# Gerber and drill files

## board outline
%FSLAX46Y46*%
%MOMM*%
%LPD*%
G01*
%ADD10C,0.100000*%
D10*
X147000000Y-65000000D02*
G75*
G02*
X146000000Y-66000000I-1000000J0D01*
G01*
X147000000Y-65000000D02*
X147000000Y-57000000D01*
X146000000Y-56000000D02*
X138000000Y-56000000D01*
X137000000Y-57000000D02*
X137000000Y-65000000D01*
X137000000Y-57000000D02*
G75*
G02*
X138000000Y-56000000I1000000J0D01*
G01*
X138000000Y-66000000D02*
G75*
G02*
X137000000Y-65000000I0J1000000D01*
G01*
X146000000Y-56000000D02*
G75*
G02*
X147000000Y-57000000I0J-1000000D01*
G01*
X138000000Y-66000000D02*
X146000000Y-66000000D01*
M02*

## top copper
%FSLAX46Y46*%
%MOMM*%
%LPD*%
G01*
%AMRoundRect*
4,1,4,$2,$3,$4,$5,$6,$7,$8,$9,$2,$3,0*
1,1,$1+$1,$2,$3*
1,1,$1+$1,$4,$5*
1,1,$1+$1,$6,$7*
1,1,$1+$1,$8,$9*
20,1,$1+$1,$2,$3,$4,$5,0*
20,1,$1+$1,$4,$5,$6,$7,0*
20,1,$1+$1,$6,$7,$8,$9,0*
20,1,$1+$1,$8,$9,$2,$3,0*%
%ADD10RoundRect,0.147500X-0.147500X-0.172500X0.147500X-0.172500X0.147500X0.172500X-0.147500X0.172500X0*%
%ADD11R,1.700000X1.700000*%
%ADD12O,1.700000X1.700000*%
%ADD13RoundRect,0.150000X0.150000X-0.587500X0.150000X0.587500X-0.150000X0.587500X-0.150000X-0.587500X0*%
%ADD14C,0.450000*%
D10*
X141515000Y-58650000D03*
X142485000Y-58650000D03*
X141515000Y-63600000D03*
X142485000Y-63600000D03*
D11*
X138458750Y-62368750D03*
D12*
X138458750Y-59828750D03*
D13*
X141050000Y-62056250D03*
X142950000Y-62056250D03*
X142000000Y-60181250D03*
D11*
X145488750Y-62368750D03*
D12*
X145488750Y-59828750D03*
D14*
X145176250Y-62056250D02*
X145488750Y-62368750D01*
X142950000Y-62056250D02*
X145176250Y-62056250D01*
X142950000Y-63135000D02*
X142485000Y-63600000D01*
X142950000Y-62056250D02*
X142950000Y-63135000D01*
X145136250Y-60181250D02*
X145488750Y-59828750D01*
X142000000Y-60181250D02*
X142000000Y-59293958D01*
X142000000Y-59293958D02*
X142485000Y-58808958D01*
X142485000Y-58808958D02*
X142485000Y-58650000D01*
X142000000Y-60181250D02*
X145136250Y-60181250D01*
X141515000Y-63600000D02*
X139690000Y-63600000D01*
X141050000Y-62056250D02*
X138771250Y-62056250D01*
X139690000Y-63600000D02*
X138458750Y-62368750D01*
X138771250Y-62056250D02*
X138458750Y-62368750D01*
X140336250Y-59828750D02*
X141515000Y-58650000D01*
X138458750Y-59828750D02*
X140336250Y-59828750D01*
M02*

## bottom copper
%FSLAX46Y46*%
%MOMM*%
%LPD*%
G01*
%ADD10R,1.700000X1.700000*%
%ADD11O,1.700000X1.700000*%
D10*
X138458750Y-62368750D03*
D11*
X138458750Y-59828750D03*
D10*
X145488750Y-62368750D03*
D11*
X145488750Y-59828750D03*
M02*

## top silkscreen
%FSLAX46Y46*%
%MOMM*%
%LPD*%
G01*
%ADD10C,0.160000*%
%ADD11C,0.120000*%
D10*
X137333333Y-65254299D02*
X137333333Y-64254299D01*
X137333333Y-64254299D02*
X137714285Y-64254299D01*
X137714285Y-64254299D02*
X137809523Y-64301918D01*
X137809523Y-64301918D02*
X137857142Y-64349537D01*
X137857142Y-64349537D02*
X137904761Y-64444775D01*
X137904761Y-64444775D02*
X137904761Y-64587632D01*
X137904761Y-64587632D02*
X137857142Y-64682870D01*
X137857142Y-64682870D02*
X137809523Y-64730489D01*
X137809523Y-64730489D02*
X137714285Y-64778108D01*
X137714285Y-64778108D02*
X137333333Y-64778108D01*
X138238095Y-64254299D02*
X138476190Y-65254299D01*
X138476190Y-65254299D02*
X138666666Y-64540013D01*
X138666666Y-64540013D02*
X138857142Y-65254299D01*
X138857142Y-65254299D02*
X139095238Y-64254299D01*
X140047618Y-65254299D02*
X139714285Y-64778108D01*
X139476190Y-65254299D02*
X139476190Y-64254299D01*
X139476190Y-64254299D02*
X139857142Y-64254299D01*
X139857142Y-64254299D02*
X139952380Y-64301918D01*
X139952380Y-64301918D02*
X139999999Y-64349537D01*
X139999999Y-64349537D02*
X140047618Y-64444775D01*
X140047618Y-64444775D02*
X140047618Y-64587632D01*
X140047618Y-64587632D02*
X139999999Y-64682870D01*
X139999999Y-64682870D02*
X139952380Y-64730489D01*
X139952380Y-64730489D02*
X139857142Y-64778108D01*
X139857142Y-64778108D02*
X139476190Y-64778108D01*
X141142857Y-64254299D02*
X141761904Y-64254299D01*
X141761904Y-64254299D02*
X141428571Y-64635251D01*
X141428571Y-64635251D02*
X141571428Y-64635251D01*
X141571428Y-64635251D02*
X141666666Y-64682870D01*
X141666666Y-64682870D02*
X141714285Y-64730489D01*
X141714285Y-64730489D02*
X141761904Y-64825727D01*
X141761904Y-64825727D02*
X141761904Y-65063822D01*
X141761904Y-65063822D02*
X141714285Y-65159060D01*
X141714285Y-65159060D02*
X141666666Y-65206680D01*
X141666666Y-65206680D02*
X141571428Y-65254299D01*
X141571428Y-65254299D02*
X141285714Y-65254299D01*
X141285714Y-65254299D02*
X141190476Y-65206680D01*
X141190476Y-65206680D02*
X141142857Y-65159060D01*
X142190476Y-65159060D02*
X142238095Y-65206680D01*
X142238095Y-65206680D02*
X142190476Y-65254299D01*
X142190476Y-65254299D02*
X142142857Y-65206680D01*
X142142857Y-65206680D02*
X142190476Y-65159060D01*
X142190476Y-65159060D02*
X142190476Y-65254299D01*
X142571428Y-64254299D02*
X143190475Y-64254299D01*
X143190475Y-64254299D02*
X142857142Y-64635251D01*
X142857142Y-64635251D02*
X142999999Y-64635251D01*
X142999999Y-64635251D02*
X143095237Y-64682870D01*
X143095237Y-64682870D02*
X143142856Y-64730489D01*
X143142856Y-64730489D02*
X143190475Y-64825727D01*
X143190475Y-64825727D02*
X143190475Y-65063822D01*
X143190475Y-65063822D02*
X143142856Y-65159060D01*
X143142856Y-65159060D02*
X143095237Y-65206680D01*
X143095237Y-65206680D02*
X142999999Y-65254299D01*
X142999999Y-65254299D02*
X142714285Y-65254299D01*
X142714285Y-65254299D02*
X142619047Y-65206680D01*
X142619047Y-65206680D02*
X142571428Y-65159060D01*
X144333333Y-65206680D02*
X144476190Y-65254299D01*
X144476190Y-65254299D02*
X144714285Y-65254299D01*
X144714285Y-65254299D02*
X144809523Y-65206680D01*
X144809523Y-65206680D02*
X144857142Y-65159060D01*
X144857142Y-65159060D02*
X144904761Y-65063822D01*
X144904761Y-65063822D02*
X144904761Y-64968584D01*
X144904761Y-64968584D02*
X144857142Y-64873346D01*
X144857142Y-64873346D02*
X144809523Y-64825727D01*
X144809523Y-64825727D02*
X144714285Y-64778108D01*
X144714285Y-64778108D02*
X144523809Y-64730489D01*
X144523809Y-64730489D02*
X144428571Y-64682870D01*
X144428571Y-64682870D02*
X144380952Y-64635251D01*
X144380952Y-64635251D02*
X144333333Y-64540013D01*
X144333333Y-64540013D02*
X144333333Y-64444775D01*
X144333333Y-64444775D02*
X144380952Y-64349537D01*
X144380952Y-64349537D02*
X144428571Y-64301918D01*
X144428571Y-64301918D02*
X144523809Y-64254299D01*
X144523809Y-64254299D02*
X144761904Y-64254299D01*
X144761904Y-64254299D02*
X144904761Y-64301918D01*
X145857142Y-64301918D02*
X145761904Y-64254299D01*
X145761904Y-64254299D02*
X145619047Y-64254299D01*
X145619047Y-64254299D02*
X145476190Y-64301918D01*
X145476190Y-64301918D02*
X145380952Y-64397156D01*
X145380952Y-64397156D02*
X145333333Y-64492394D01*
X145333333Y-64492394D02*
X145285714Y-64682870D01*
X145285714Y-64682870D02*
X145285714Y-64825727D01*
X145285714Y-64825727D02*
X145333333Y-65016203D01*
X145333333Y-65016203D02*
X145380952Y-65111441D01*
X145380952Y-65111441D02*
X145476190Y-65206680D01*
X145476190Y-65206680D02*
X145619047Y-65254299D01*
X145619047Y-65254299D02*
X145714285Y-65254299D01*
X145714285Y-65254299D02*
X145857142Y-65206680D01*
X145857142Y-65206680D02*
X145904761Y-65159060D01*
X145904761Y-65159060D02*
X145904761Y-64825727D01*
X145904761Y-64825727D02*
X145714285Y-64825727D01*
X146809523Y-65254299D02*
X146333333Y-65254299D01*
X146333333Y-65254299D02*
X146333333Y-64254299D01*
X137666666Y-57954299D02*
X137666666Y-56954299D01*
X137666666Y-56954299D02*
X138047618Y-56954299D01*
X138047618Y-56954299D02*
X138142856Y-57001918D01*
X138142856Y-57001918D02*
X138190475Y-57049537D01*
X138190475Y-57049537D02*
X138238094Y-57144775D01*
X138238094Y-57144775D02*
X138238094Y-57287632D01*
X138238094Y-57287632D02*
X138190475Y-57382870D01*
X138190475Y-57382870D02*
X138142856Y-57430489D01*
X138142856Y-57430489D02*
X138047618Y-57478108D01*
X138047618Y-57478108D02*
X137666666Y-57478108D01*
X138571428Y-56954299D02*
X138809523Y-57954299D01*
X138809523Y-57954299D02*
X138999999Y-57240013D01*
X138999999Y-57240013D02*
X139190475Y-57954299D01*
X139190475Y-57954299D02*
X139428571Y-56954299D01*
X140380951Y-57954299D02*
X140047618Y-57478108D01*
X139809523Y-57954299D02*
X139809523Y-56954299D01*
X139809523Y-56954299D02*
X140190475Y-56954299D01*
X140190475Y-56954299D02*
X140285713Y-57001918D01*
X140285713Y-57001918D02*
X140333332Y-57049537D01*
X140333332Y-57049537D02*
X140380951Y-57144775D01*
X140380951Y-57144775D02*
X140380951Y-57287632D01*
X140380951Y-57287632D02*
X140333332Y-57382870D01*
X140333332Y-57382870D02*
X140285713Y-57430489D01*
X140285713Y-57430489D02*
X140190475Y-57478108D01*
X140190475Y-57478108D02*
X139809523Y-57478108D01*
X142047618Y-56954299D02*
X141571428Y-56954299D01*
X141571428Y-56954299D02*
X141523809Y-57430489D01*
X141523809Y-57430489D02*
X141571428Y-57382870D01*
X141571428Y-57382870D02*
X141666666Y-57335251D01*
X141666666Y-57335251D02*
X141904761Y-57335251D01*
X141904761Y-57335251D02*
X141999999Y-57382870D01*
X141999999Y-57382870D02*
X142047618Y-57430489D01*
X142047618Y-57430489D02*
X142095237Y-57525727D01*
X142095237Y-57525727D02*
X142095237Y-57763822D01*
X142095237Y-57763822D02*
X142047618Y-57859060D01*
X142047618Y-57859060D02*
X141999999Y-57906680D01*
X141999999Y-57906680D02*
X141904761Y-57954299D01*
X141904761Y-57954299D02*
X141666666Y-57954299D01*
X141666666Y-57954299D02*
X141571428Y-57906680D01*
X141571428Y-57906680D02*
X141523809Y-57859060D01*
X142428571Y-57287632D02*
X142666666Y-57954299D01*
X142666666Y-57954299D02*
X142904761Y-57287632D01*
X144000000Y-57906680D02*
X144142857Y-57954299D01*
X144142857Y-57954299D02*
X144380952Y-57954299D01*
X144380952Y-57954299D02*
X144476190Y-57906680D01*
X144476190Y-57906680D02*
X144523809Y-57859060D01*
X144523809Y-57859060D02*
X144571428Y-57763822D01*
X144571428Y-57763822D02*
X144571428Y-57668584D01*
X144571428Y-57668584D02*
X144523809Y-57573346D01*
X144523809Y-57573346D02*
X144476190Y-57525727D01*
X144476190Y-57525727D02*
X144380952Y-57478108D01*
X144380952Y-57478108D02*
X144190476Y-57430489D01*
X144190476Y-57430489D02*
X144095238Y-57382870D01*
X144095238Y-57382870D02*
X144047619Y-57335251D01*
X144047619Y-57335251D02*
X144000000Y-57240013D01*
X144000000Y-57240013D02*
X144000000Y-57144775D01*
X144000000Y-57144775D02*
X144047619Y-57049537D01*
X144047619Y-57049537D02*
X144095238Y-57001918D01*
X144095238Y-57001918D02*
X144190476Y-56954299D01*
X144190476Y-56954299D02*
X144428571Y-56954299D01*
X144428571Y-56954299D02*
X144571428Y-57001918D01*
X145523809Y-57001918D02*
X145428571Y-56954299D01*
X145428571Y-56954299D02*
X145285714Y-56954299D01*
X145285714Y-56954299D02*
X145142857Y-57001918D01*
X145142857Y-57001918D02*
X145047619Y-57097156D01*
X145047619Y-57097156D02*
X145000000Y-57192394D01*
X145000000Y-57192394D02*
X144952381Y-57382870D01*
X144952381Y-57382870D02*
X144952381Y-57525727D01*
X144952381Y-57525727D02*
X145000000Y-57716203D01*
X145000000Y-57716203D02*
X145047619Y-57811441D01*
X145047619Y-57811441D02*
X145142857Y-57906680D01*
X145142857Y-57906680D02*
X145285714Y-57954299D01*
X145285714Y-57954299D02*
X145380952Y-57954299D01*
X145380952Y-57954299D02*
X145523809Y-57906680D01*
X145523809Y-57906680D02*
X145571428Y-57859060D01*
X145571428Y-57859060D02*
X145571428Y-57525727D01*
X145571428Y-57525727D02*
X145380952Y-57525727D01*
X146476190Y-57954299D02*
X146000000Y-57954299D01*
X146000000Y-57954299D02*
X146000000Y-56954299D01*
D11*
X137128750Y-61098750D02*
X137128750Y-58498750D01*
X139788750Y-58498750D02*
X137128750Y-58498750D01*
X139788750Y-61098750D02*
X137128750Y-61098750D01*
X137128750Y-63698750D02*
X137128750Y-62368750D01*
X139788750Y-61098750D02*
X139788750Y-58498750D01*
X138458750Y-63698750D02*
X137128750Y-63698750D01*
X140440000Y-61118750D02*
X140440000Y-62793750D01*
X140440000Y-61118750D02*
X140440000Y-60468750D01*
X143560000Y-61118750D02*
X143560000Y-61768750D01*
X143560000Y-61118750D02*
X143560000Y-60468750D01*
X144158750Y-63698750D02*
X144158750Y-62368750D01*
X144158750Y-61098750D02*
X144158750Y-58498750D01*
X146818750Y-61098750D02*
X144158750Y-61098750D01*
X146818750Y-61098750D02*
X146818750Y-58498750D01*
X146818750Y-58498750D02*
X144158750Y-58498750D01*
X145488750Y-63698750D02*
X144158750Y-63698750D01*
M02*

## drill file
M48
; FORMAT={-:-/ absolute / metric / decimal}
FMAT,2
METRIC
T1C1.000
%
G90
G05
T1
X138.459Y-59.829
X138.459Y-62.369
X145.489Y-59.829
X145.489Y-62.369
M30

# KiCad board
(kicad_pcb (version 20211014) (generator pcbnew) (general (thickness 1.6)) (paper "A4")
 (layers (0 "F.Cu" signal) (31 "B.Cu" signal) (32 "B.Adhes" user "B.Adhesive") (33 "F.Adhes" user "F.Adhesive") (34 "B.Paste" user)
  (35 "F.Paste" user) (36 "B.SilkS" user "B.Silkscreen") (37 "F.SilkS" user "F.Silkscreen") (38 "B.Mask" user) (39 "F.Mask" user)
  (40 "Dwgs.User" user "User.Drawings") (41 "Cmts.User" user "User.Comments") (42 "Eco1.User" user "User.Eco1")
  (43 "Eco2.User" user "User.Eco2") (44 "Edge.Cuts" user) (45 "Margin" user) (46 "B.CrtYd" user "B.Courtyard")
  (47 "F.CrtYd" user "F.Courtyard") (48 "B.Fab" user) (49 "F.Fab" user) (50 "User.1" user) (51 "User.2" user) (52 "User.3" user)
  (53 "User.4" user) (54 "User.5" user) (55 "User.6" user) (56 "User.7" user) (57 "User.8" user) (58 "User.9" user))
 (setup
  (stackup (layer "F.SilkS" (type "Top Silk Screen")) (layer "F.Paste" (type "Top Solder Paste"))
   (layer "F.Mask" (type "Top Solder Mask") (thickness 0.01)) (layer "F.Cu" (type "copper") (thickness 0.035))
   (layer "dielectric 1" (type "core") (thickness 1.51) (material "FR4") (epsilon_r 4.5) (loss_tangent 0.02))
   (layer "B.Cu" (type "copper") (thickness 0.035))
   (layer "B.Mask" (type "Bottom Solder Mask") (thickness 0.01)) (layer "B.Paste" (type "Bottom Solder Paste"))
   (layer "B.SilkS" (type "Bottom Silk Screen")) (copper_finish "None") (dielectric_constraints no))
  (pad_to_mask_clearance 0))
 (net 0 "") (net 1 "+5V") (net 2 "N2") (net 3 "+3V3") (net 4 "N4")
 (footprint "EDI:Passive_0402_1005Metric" (layer "F.Cu") (at 142 58.65)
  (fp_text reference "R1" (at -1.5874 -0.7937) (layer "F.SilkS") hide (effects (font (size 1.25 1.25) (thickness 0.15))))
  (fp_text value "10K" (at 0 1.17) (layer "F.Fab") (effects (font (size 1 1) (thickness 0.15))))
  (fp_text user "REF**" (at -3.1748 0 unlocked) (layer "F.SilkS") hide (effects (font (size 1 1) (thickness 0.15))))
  (pad "1" smd roundrect (at -0.485 0) (size 0.59 0.64) (layers "F.Cu" "F.Paste" "F.Mask") (roundrect_rratio 0.25) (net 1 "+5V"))
  (pad "2" smd roundrect (at 0.485 0) (size 0.59 0.64) (layers "F.Cu" "F.Paste" "F.Mask") (roundrect_rratio 0.25) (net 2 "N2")))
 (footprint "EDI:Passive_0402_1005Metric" (layer "F.Cu") (at 142 63.6)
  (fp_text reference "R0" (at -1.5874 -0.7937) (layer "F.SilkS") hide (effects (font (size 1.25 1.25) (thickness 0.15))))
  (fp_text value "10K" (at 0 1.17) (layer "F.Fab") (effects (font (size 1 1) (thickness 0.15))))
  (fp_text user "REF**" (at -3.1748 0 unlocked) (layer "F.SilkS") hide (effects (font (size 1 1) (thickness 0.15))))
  (pad "1" smd roundrect (at -0.485 0) (size 0.59 0.64) (layers "F.Cu" "F.Paste" "F.Mask") (roundrect_rratio 0.25) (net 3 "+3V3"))
  (pad "2" smd roundrect (at 0.485 0) (size 0.59 0.64) (layers "F.Cu" "F.Paste" "F.Mask") (roundrect_rratio 0.25) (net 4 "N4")))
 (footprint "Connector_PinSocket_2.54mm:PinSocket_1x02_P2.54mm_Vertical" (layer "F.Cu") (at 138.45875 62.36875 180)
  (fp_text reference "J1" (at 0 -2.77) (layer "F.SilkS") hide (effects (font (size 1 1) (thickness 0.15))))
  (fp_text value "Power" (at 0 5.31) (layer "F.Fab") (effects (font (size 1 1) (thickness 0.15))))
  (fp_line (start 1.33 1.27) (end 1.33 3.87) (layer "F.SilkS") (width 0.12))
  (fp_line (start -1.33 3.87) (end 1.33 3.87) (layer "F.SilkS") (width 0.12))
  (fp_line (start -1.33 1.27) (end 1.33 1.27) (layer "F.SilkS") (width 0.12))
  (fp_line (start 1.33 -1.33) (end 1.33 0) (layer "F.SilkS") (width 0.12))
  (fp_line (start -1.33 1.27) (end -1.33 3.87) (layer "F.SilkS") (width 0.12))
  (fp_line (start 0 -1.33) (end 1.33 -1.33) (layer "F.SilkS") (width 0.12))
  (pad "1" thru_hole rect locked (at 0 0 180) (size 1.7 1.7) (drill 1) (layers *.Cu *.Mask) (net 3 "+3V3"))
  (pad "2" thru_hole oval locked (at 0 2.54 180) (size 1.7 1.7) (drill 1) (layers *.Cu *.Mask) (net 1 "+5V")))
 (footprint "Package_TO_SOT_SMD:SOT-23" (layer "F.Cu") (at 142 61.11875 90)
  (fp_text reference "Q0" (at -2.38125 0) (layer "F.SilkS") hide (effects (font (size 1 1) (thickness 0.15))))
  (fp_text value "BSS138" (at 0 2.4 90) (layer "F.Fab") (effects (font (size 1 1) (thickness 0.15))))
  (fp_line (start 0 -1.56) (end -1.675 -1.56) (layer "F.SilkS") (width 0.12))
  (fp_line (start 0 -1.56) (end 0.65 -1.56) (layer "F.SilkS") (width 0.12))
  (fp_line (start 0 1.56) (end -0.65 1.56) (layer "F.SilkS") (width 0.12))
  (fp_line (start 0 1.56) (end 0.65 1.56) (layer "F.SilkS") (width 0.12))
  (pad "1" smd roundrect locked (at -0.9375 -0.95 90) (size 1.475 0.6) (layers "F.Cu" "F.Paste" "F.Mask") (roundrect_rratio 0.25)
   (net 3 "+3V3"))
  (pad "2" smd roundrect locked (at -0.9375 0.95 90) (size 1.475 0.6) (layers "F.Cu" "F.Paste" "F.Mask") (roundrect_rratio 0.25)
   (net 4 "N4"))
  (pad "3" smd roundrect locked (at 0.9375 0 90) (size 1.475 0.6) (layers "F.Cu" "F.Paste" "F.Mask") (roundrect_rratio 0.25) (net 2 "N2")))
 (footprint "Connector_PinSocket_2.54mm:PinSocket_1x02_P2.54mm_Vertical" (layer "F.Cu") (at 145.48875 62.36875 180)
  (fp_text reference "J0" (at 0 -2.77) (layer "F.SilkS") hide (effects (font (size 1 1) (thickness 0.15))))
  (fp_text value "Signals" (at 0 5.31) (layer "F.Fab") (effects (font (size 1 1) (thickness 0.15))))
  (fp_line (start 1.33 -1.33) (end 1.33 0) (layer "F.SilkS") (width 0.12))
  (fp_line (start 1.33 1.27) (end 1.33 3.87) (layer "F.SilkS") (width 0.12))
  (fp_line (start -1.33 1.27) (end 1.33 1.27) (layer "F.SilkS") (width 0.12))
  (fp_line (start -1.33 1.27) (end -1.33 3.87) (layer "F.SilkS") (width 0.12))
  (fp_line (start -1.33 3.87) (end 1.33 3.87) (layer "F.SilkS") (width 0.12))
  (fp_line (start 0 -1.33) (end 1.33 -1.33) (layer "F.SilkS") (width 0.12))
  (pad "1" thru_hole rect locked (at 0 0 180) (size 1.7 1.7) (drill 1) (layers *.Cu *.Mask) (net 4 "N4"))
  (pad "2" thru_hole oval locked (at 0 2.54 180) (size 1.7 1.7) (drill 1) (layers *.Cu *.Mask) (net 2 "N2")))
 (gr_arc (start 147 65) (mid 146.707107 65.707107) (end 146 66) (layer "Edge.Cuts") (width 0.1))
 (gr_line (start 147 65) (end 147 57) (layer "Edge.Cuts") (width 0.1))
 (gr_line (start 146 56) (end 138 56) (layer "Edge.Cuts") (width 0.1))
 (gr_line (start 137 57) (end 137 65) (layer "Edge.Cuts") (width 0.1))
 (gr_arc (start 137 57) (mid 137.292893 56.292893) (end 138 56) (layer "Edge.Cuts") (width 0.1))
 (gr_arc (start 138 66) (mid 137.292893 65.707107) (end 137 65) (layer "Edge.Cuts") (width 0.1))
 (gr_arc (start 146 56) (mid 146.707107 56.292893) (end 147 57) (layer "Edge.Cuts") (width 0.1))
 (gr_line (start 138 66) (end 146 66) (layer "Edge.Cuts") (width 0.1))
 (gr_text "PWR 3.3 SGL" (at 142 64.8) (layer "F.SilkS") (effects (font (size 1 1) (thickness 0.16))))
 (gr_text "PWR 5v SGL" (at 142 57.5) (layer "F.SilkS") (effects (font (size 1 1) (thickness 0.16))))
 (segment (start 145.17625 62.05625) (end 145.48875 62.36875) (width 0.45) (layer "F.Cu") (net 4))
 (segment (start 142.95 62.05625) (end 145.17625 62.05625) (width 0.45) (layer "F.Cu") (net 4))
 (segment (start 142.95 63.135) (end 142.485 63.6) (width 0.45) (layer "F.Cu") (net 4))
 (segment (start 142.95 62.05625) (end 142.95 63.135) (width 0.45) (layer "F.Cu") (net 4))
 (segment (start 145.13625 60.18125) (end 145.48875 59.82875) (width 0.45) (layer "F.Cu") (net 2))
 (segment (start 142 60.18125) (end 142 59.293958) (width 0.45) (layer "F.Cu") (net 2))
 (segment (start 142 59.293958) (end 142.485 58.808958) (width 0.45) (layer "F.Cu") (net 2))
 (segment (start 142.485 58.808958) (end 142.485 58.65) (width 0.45) (layer "F.Cu") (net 2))
 (segment (start 142 60.18125) (end 145.13625 60.18125) (width 0.45) (layer "F.Cu") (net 2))
 (segment (start 141.515 63.6) (end 139.69 63.6) (width 0.45) (layer "F.Cu") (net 3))
 (segment (start 141.05 62.05625) (end 138.77125 62.05625) (width 0.45) (layer "F.Cu") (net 3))
 (segment (start 139.69 63.6) (end 138.45875 62.36875) (width 0.45) (layer "F.Cu") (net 3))
 (segment (start 138.77125 62.05625) (end 138.45875 62.36875) (width 0.45) (layer "F.Cu") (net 3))
 (segment (start 140.33625 59.82875) (end 141.515 58.65) (width 0.45) (layer "F.Cu") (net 1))
 (segment (start 138.45875 59.82875) (end 140.33625 59.82875) (width 0.45) (layer "F.Cu") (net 1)))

